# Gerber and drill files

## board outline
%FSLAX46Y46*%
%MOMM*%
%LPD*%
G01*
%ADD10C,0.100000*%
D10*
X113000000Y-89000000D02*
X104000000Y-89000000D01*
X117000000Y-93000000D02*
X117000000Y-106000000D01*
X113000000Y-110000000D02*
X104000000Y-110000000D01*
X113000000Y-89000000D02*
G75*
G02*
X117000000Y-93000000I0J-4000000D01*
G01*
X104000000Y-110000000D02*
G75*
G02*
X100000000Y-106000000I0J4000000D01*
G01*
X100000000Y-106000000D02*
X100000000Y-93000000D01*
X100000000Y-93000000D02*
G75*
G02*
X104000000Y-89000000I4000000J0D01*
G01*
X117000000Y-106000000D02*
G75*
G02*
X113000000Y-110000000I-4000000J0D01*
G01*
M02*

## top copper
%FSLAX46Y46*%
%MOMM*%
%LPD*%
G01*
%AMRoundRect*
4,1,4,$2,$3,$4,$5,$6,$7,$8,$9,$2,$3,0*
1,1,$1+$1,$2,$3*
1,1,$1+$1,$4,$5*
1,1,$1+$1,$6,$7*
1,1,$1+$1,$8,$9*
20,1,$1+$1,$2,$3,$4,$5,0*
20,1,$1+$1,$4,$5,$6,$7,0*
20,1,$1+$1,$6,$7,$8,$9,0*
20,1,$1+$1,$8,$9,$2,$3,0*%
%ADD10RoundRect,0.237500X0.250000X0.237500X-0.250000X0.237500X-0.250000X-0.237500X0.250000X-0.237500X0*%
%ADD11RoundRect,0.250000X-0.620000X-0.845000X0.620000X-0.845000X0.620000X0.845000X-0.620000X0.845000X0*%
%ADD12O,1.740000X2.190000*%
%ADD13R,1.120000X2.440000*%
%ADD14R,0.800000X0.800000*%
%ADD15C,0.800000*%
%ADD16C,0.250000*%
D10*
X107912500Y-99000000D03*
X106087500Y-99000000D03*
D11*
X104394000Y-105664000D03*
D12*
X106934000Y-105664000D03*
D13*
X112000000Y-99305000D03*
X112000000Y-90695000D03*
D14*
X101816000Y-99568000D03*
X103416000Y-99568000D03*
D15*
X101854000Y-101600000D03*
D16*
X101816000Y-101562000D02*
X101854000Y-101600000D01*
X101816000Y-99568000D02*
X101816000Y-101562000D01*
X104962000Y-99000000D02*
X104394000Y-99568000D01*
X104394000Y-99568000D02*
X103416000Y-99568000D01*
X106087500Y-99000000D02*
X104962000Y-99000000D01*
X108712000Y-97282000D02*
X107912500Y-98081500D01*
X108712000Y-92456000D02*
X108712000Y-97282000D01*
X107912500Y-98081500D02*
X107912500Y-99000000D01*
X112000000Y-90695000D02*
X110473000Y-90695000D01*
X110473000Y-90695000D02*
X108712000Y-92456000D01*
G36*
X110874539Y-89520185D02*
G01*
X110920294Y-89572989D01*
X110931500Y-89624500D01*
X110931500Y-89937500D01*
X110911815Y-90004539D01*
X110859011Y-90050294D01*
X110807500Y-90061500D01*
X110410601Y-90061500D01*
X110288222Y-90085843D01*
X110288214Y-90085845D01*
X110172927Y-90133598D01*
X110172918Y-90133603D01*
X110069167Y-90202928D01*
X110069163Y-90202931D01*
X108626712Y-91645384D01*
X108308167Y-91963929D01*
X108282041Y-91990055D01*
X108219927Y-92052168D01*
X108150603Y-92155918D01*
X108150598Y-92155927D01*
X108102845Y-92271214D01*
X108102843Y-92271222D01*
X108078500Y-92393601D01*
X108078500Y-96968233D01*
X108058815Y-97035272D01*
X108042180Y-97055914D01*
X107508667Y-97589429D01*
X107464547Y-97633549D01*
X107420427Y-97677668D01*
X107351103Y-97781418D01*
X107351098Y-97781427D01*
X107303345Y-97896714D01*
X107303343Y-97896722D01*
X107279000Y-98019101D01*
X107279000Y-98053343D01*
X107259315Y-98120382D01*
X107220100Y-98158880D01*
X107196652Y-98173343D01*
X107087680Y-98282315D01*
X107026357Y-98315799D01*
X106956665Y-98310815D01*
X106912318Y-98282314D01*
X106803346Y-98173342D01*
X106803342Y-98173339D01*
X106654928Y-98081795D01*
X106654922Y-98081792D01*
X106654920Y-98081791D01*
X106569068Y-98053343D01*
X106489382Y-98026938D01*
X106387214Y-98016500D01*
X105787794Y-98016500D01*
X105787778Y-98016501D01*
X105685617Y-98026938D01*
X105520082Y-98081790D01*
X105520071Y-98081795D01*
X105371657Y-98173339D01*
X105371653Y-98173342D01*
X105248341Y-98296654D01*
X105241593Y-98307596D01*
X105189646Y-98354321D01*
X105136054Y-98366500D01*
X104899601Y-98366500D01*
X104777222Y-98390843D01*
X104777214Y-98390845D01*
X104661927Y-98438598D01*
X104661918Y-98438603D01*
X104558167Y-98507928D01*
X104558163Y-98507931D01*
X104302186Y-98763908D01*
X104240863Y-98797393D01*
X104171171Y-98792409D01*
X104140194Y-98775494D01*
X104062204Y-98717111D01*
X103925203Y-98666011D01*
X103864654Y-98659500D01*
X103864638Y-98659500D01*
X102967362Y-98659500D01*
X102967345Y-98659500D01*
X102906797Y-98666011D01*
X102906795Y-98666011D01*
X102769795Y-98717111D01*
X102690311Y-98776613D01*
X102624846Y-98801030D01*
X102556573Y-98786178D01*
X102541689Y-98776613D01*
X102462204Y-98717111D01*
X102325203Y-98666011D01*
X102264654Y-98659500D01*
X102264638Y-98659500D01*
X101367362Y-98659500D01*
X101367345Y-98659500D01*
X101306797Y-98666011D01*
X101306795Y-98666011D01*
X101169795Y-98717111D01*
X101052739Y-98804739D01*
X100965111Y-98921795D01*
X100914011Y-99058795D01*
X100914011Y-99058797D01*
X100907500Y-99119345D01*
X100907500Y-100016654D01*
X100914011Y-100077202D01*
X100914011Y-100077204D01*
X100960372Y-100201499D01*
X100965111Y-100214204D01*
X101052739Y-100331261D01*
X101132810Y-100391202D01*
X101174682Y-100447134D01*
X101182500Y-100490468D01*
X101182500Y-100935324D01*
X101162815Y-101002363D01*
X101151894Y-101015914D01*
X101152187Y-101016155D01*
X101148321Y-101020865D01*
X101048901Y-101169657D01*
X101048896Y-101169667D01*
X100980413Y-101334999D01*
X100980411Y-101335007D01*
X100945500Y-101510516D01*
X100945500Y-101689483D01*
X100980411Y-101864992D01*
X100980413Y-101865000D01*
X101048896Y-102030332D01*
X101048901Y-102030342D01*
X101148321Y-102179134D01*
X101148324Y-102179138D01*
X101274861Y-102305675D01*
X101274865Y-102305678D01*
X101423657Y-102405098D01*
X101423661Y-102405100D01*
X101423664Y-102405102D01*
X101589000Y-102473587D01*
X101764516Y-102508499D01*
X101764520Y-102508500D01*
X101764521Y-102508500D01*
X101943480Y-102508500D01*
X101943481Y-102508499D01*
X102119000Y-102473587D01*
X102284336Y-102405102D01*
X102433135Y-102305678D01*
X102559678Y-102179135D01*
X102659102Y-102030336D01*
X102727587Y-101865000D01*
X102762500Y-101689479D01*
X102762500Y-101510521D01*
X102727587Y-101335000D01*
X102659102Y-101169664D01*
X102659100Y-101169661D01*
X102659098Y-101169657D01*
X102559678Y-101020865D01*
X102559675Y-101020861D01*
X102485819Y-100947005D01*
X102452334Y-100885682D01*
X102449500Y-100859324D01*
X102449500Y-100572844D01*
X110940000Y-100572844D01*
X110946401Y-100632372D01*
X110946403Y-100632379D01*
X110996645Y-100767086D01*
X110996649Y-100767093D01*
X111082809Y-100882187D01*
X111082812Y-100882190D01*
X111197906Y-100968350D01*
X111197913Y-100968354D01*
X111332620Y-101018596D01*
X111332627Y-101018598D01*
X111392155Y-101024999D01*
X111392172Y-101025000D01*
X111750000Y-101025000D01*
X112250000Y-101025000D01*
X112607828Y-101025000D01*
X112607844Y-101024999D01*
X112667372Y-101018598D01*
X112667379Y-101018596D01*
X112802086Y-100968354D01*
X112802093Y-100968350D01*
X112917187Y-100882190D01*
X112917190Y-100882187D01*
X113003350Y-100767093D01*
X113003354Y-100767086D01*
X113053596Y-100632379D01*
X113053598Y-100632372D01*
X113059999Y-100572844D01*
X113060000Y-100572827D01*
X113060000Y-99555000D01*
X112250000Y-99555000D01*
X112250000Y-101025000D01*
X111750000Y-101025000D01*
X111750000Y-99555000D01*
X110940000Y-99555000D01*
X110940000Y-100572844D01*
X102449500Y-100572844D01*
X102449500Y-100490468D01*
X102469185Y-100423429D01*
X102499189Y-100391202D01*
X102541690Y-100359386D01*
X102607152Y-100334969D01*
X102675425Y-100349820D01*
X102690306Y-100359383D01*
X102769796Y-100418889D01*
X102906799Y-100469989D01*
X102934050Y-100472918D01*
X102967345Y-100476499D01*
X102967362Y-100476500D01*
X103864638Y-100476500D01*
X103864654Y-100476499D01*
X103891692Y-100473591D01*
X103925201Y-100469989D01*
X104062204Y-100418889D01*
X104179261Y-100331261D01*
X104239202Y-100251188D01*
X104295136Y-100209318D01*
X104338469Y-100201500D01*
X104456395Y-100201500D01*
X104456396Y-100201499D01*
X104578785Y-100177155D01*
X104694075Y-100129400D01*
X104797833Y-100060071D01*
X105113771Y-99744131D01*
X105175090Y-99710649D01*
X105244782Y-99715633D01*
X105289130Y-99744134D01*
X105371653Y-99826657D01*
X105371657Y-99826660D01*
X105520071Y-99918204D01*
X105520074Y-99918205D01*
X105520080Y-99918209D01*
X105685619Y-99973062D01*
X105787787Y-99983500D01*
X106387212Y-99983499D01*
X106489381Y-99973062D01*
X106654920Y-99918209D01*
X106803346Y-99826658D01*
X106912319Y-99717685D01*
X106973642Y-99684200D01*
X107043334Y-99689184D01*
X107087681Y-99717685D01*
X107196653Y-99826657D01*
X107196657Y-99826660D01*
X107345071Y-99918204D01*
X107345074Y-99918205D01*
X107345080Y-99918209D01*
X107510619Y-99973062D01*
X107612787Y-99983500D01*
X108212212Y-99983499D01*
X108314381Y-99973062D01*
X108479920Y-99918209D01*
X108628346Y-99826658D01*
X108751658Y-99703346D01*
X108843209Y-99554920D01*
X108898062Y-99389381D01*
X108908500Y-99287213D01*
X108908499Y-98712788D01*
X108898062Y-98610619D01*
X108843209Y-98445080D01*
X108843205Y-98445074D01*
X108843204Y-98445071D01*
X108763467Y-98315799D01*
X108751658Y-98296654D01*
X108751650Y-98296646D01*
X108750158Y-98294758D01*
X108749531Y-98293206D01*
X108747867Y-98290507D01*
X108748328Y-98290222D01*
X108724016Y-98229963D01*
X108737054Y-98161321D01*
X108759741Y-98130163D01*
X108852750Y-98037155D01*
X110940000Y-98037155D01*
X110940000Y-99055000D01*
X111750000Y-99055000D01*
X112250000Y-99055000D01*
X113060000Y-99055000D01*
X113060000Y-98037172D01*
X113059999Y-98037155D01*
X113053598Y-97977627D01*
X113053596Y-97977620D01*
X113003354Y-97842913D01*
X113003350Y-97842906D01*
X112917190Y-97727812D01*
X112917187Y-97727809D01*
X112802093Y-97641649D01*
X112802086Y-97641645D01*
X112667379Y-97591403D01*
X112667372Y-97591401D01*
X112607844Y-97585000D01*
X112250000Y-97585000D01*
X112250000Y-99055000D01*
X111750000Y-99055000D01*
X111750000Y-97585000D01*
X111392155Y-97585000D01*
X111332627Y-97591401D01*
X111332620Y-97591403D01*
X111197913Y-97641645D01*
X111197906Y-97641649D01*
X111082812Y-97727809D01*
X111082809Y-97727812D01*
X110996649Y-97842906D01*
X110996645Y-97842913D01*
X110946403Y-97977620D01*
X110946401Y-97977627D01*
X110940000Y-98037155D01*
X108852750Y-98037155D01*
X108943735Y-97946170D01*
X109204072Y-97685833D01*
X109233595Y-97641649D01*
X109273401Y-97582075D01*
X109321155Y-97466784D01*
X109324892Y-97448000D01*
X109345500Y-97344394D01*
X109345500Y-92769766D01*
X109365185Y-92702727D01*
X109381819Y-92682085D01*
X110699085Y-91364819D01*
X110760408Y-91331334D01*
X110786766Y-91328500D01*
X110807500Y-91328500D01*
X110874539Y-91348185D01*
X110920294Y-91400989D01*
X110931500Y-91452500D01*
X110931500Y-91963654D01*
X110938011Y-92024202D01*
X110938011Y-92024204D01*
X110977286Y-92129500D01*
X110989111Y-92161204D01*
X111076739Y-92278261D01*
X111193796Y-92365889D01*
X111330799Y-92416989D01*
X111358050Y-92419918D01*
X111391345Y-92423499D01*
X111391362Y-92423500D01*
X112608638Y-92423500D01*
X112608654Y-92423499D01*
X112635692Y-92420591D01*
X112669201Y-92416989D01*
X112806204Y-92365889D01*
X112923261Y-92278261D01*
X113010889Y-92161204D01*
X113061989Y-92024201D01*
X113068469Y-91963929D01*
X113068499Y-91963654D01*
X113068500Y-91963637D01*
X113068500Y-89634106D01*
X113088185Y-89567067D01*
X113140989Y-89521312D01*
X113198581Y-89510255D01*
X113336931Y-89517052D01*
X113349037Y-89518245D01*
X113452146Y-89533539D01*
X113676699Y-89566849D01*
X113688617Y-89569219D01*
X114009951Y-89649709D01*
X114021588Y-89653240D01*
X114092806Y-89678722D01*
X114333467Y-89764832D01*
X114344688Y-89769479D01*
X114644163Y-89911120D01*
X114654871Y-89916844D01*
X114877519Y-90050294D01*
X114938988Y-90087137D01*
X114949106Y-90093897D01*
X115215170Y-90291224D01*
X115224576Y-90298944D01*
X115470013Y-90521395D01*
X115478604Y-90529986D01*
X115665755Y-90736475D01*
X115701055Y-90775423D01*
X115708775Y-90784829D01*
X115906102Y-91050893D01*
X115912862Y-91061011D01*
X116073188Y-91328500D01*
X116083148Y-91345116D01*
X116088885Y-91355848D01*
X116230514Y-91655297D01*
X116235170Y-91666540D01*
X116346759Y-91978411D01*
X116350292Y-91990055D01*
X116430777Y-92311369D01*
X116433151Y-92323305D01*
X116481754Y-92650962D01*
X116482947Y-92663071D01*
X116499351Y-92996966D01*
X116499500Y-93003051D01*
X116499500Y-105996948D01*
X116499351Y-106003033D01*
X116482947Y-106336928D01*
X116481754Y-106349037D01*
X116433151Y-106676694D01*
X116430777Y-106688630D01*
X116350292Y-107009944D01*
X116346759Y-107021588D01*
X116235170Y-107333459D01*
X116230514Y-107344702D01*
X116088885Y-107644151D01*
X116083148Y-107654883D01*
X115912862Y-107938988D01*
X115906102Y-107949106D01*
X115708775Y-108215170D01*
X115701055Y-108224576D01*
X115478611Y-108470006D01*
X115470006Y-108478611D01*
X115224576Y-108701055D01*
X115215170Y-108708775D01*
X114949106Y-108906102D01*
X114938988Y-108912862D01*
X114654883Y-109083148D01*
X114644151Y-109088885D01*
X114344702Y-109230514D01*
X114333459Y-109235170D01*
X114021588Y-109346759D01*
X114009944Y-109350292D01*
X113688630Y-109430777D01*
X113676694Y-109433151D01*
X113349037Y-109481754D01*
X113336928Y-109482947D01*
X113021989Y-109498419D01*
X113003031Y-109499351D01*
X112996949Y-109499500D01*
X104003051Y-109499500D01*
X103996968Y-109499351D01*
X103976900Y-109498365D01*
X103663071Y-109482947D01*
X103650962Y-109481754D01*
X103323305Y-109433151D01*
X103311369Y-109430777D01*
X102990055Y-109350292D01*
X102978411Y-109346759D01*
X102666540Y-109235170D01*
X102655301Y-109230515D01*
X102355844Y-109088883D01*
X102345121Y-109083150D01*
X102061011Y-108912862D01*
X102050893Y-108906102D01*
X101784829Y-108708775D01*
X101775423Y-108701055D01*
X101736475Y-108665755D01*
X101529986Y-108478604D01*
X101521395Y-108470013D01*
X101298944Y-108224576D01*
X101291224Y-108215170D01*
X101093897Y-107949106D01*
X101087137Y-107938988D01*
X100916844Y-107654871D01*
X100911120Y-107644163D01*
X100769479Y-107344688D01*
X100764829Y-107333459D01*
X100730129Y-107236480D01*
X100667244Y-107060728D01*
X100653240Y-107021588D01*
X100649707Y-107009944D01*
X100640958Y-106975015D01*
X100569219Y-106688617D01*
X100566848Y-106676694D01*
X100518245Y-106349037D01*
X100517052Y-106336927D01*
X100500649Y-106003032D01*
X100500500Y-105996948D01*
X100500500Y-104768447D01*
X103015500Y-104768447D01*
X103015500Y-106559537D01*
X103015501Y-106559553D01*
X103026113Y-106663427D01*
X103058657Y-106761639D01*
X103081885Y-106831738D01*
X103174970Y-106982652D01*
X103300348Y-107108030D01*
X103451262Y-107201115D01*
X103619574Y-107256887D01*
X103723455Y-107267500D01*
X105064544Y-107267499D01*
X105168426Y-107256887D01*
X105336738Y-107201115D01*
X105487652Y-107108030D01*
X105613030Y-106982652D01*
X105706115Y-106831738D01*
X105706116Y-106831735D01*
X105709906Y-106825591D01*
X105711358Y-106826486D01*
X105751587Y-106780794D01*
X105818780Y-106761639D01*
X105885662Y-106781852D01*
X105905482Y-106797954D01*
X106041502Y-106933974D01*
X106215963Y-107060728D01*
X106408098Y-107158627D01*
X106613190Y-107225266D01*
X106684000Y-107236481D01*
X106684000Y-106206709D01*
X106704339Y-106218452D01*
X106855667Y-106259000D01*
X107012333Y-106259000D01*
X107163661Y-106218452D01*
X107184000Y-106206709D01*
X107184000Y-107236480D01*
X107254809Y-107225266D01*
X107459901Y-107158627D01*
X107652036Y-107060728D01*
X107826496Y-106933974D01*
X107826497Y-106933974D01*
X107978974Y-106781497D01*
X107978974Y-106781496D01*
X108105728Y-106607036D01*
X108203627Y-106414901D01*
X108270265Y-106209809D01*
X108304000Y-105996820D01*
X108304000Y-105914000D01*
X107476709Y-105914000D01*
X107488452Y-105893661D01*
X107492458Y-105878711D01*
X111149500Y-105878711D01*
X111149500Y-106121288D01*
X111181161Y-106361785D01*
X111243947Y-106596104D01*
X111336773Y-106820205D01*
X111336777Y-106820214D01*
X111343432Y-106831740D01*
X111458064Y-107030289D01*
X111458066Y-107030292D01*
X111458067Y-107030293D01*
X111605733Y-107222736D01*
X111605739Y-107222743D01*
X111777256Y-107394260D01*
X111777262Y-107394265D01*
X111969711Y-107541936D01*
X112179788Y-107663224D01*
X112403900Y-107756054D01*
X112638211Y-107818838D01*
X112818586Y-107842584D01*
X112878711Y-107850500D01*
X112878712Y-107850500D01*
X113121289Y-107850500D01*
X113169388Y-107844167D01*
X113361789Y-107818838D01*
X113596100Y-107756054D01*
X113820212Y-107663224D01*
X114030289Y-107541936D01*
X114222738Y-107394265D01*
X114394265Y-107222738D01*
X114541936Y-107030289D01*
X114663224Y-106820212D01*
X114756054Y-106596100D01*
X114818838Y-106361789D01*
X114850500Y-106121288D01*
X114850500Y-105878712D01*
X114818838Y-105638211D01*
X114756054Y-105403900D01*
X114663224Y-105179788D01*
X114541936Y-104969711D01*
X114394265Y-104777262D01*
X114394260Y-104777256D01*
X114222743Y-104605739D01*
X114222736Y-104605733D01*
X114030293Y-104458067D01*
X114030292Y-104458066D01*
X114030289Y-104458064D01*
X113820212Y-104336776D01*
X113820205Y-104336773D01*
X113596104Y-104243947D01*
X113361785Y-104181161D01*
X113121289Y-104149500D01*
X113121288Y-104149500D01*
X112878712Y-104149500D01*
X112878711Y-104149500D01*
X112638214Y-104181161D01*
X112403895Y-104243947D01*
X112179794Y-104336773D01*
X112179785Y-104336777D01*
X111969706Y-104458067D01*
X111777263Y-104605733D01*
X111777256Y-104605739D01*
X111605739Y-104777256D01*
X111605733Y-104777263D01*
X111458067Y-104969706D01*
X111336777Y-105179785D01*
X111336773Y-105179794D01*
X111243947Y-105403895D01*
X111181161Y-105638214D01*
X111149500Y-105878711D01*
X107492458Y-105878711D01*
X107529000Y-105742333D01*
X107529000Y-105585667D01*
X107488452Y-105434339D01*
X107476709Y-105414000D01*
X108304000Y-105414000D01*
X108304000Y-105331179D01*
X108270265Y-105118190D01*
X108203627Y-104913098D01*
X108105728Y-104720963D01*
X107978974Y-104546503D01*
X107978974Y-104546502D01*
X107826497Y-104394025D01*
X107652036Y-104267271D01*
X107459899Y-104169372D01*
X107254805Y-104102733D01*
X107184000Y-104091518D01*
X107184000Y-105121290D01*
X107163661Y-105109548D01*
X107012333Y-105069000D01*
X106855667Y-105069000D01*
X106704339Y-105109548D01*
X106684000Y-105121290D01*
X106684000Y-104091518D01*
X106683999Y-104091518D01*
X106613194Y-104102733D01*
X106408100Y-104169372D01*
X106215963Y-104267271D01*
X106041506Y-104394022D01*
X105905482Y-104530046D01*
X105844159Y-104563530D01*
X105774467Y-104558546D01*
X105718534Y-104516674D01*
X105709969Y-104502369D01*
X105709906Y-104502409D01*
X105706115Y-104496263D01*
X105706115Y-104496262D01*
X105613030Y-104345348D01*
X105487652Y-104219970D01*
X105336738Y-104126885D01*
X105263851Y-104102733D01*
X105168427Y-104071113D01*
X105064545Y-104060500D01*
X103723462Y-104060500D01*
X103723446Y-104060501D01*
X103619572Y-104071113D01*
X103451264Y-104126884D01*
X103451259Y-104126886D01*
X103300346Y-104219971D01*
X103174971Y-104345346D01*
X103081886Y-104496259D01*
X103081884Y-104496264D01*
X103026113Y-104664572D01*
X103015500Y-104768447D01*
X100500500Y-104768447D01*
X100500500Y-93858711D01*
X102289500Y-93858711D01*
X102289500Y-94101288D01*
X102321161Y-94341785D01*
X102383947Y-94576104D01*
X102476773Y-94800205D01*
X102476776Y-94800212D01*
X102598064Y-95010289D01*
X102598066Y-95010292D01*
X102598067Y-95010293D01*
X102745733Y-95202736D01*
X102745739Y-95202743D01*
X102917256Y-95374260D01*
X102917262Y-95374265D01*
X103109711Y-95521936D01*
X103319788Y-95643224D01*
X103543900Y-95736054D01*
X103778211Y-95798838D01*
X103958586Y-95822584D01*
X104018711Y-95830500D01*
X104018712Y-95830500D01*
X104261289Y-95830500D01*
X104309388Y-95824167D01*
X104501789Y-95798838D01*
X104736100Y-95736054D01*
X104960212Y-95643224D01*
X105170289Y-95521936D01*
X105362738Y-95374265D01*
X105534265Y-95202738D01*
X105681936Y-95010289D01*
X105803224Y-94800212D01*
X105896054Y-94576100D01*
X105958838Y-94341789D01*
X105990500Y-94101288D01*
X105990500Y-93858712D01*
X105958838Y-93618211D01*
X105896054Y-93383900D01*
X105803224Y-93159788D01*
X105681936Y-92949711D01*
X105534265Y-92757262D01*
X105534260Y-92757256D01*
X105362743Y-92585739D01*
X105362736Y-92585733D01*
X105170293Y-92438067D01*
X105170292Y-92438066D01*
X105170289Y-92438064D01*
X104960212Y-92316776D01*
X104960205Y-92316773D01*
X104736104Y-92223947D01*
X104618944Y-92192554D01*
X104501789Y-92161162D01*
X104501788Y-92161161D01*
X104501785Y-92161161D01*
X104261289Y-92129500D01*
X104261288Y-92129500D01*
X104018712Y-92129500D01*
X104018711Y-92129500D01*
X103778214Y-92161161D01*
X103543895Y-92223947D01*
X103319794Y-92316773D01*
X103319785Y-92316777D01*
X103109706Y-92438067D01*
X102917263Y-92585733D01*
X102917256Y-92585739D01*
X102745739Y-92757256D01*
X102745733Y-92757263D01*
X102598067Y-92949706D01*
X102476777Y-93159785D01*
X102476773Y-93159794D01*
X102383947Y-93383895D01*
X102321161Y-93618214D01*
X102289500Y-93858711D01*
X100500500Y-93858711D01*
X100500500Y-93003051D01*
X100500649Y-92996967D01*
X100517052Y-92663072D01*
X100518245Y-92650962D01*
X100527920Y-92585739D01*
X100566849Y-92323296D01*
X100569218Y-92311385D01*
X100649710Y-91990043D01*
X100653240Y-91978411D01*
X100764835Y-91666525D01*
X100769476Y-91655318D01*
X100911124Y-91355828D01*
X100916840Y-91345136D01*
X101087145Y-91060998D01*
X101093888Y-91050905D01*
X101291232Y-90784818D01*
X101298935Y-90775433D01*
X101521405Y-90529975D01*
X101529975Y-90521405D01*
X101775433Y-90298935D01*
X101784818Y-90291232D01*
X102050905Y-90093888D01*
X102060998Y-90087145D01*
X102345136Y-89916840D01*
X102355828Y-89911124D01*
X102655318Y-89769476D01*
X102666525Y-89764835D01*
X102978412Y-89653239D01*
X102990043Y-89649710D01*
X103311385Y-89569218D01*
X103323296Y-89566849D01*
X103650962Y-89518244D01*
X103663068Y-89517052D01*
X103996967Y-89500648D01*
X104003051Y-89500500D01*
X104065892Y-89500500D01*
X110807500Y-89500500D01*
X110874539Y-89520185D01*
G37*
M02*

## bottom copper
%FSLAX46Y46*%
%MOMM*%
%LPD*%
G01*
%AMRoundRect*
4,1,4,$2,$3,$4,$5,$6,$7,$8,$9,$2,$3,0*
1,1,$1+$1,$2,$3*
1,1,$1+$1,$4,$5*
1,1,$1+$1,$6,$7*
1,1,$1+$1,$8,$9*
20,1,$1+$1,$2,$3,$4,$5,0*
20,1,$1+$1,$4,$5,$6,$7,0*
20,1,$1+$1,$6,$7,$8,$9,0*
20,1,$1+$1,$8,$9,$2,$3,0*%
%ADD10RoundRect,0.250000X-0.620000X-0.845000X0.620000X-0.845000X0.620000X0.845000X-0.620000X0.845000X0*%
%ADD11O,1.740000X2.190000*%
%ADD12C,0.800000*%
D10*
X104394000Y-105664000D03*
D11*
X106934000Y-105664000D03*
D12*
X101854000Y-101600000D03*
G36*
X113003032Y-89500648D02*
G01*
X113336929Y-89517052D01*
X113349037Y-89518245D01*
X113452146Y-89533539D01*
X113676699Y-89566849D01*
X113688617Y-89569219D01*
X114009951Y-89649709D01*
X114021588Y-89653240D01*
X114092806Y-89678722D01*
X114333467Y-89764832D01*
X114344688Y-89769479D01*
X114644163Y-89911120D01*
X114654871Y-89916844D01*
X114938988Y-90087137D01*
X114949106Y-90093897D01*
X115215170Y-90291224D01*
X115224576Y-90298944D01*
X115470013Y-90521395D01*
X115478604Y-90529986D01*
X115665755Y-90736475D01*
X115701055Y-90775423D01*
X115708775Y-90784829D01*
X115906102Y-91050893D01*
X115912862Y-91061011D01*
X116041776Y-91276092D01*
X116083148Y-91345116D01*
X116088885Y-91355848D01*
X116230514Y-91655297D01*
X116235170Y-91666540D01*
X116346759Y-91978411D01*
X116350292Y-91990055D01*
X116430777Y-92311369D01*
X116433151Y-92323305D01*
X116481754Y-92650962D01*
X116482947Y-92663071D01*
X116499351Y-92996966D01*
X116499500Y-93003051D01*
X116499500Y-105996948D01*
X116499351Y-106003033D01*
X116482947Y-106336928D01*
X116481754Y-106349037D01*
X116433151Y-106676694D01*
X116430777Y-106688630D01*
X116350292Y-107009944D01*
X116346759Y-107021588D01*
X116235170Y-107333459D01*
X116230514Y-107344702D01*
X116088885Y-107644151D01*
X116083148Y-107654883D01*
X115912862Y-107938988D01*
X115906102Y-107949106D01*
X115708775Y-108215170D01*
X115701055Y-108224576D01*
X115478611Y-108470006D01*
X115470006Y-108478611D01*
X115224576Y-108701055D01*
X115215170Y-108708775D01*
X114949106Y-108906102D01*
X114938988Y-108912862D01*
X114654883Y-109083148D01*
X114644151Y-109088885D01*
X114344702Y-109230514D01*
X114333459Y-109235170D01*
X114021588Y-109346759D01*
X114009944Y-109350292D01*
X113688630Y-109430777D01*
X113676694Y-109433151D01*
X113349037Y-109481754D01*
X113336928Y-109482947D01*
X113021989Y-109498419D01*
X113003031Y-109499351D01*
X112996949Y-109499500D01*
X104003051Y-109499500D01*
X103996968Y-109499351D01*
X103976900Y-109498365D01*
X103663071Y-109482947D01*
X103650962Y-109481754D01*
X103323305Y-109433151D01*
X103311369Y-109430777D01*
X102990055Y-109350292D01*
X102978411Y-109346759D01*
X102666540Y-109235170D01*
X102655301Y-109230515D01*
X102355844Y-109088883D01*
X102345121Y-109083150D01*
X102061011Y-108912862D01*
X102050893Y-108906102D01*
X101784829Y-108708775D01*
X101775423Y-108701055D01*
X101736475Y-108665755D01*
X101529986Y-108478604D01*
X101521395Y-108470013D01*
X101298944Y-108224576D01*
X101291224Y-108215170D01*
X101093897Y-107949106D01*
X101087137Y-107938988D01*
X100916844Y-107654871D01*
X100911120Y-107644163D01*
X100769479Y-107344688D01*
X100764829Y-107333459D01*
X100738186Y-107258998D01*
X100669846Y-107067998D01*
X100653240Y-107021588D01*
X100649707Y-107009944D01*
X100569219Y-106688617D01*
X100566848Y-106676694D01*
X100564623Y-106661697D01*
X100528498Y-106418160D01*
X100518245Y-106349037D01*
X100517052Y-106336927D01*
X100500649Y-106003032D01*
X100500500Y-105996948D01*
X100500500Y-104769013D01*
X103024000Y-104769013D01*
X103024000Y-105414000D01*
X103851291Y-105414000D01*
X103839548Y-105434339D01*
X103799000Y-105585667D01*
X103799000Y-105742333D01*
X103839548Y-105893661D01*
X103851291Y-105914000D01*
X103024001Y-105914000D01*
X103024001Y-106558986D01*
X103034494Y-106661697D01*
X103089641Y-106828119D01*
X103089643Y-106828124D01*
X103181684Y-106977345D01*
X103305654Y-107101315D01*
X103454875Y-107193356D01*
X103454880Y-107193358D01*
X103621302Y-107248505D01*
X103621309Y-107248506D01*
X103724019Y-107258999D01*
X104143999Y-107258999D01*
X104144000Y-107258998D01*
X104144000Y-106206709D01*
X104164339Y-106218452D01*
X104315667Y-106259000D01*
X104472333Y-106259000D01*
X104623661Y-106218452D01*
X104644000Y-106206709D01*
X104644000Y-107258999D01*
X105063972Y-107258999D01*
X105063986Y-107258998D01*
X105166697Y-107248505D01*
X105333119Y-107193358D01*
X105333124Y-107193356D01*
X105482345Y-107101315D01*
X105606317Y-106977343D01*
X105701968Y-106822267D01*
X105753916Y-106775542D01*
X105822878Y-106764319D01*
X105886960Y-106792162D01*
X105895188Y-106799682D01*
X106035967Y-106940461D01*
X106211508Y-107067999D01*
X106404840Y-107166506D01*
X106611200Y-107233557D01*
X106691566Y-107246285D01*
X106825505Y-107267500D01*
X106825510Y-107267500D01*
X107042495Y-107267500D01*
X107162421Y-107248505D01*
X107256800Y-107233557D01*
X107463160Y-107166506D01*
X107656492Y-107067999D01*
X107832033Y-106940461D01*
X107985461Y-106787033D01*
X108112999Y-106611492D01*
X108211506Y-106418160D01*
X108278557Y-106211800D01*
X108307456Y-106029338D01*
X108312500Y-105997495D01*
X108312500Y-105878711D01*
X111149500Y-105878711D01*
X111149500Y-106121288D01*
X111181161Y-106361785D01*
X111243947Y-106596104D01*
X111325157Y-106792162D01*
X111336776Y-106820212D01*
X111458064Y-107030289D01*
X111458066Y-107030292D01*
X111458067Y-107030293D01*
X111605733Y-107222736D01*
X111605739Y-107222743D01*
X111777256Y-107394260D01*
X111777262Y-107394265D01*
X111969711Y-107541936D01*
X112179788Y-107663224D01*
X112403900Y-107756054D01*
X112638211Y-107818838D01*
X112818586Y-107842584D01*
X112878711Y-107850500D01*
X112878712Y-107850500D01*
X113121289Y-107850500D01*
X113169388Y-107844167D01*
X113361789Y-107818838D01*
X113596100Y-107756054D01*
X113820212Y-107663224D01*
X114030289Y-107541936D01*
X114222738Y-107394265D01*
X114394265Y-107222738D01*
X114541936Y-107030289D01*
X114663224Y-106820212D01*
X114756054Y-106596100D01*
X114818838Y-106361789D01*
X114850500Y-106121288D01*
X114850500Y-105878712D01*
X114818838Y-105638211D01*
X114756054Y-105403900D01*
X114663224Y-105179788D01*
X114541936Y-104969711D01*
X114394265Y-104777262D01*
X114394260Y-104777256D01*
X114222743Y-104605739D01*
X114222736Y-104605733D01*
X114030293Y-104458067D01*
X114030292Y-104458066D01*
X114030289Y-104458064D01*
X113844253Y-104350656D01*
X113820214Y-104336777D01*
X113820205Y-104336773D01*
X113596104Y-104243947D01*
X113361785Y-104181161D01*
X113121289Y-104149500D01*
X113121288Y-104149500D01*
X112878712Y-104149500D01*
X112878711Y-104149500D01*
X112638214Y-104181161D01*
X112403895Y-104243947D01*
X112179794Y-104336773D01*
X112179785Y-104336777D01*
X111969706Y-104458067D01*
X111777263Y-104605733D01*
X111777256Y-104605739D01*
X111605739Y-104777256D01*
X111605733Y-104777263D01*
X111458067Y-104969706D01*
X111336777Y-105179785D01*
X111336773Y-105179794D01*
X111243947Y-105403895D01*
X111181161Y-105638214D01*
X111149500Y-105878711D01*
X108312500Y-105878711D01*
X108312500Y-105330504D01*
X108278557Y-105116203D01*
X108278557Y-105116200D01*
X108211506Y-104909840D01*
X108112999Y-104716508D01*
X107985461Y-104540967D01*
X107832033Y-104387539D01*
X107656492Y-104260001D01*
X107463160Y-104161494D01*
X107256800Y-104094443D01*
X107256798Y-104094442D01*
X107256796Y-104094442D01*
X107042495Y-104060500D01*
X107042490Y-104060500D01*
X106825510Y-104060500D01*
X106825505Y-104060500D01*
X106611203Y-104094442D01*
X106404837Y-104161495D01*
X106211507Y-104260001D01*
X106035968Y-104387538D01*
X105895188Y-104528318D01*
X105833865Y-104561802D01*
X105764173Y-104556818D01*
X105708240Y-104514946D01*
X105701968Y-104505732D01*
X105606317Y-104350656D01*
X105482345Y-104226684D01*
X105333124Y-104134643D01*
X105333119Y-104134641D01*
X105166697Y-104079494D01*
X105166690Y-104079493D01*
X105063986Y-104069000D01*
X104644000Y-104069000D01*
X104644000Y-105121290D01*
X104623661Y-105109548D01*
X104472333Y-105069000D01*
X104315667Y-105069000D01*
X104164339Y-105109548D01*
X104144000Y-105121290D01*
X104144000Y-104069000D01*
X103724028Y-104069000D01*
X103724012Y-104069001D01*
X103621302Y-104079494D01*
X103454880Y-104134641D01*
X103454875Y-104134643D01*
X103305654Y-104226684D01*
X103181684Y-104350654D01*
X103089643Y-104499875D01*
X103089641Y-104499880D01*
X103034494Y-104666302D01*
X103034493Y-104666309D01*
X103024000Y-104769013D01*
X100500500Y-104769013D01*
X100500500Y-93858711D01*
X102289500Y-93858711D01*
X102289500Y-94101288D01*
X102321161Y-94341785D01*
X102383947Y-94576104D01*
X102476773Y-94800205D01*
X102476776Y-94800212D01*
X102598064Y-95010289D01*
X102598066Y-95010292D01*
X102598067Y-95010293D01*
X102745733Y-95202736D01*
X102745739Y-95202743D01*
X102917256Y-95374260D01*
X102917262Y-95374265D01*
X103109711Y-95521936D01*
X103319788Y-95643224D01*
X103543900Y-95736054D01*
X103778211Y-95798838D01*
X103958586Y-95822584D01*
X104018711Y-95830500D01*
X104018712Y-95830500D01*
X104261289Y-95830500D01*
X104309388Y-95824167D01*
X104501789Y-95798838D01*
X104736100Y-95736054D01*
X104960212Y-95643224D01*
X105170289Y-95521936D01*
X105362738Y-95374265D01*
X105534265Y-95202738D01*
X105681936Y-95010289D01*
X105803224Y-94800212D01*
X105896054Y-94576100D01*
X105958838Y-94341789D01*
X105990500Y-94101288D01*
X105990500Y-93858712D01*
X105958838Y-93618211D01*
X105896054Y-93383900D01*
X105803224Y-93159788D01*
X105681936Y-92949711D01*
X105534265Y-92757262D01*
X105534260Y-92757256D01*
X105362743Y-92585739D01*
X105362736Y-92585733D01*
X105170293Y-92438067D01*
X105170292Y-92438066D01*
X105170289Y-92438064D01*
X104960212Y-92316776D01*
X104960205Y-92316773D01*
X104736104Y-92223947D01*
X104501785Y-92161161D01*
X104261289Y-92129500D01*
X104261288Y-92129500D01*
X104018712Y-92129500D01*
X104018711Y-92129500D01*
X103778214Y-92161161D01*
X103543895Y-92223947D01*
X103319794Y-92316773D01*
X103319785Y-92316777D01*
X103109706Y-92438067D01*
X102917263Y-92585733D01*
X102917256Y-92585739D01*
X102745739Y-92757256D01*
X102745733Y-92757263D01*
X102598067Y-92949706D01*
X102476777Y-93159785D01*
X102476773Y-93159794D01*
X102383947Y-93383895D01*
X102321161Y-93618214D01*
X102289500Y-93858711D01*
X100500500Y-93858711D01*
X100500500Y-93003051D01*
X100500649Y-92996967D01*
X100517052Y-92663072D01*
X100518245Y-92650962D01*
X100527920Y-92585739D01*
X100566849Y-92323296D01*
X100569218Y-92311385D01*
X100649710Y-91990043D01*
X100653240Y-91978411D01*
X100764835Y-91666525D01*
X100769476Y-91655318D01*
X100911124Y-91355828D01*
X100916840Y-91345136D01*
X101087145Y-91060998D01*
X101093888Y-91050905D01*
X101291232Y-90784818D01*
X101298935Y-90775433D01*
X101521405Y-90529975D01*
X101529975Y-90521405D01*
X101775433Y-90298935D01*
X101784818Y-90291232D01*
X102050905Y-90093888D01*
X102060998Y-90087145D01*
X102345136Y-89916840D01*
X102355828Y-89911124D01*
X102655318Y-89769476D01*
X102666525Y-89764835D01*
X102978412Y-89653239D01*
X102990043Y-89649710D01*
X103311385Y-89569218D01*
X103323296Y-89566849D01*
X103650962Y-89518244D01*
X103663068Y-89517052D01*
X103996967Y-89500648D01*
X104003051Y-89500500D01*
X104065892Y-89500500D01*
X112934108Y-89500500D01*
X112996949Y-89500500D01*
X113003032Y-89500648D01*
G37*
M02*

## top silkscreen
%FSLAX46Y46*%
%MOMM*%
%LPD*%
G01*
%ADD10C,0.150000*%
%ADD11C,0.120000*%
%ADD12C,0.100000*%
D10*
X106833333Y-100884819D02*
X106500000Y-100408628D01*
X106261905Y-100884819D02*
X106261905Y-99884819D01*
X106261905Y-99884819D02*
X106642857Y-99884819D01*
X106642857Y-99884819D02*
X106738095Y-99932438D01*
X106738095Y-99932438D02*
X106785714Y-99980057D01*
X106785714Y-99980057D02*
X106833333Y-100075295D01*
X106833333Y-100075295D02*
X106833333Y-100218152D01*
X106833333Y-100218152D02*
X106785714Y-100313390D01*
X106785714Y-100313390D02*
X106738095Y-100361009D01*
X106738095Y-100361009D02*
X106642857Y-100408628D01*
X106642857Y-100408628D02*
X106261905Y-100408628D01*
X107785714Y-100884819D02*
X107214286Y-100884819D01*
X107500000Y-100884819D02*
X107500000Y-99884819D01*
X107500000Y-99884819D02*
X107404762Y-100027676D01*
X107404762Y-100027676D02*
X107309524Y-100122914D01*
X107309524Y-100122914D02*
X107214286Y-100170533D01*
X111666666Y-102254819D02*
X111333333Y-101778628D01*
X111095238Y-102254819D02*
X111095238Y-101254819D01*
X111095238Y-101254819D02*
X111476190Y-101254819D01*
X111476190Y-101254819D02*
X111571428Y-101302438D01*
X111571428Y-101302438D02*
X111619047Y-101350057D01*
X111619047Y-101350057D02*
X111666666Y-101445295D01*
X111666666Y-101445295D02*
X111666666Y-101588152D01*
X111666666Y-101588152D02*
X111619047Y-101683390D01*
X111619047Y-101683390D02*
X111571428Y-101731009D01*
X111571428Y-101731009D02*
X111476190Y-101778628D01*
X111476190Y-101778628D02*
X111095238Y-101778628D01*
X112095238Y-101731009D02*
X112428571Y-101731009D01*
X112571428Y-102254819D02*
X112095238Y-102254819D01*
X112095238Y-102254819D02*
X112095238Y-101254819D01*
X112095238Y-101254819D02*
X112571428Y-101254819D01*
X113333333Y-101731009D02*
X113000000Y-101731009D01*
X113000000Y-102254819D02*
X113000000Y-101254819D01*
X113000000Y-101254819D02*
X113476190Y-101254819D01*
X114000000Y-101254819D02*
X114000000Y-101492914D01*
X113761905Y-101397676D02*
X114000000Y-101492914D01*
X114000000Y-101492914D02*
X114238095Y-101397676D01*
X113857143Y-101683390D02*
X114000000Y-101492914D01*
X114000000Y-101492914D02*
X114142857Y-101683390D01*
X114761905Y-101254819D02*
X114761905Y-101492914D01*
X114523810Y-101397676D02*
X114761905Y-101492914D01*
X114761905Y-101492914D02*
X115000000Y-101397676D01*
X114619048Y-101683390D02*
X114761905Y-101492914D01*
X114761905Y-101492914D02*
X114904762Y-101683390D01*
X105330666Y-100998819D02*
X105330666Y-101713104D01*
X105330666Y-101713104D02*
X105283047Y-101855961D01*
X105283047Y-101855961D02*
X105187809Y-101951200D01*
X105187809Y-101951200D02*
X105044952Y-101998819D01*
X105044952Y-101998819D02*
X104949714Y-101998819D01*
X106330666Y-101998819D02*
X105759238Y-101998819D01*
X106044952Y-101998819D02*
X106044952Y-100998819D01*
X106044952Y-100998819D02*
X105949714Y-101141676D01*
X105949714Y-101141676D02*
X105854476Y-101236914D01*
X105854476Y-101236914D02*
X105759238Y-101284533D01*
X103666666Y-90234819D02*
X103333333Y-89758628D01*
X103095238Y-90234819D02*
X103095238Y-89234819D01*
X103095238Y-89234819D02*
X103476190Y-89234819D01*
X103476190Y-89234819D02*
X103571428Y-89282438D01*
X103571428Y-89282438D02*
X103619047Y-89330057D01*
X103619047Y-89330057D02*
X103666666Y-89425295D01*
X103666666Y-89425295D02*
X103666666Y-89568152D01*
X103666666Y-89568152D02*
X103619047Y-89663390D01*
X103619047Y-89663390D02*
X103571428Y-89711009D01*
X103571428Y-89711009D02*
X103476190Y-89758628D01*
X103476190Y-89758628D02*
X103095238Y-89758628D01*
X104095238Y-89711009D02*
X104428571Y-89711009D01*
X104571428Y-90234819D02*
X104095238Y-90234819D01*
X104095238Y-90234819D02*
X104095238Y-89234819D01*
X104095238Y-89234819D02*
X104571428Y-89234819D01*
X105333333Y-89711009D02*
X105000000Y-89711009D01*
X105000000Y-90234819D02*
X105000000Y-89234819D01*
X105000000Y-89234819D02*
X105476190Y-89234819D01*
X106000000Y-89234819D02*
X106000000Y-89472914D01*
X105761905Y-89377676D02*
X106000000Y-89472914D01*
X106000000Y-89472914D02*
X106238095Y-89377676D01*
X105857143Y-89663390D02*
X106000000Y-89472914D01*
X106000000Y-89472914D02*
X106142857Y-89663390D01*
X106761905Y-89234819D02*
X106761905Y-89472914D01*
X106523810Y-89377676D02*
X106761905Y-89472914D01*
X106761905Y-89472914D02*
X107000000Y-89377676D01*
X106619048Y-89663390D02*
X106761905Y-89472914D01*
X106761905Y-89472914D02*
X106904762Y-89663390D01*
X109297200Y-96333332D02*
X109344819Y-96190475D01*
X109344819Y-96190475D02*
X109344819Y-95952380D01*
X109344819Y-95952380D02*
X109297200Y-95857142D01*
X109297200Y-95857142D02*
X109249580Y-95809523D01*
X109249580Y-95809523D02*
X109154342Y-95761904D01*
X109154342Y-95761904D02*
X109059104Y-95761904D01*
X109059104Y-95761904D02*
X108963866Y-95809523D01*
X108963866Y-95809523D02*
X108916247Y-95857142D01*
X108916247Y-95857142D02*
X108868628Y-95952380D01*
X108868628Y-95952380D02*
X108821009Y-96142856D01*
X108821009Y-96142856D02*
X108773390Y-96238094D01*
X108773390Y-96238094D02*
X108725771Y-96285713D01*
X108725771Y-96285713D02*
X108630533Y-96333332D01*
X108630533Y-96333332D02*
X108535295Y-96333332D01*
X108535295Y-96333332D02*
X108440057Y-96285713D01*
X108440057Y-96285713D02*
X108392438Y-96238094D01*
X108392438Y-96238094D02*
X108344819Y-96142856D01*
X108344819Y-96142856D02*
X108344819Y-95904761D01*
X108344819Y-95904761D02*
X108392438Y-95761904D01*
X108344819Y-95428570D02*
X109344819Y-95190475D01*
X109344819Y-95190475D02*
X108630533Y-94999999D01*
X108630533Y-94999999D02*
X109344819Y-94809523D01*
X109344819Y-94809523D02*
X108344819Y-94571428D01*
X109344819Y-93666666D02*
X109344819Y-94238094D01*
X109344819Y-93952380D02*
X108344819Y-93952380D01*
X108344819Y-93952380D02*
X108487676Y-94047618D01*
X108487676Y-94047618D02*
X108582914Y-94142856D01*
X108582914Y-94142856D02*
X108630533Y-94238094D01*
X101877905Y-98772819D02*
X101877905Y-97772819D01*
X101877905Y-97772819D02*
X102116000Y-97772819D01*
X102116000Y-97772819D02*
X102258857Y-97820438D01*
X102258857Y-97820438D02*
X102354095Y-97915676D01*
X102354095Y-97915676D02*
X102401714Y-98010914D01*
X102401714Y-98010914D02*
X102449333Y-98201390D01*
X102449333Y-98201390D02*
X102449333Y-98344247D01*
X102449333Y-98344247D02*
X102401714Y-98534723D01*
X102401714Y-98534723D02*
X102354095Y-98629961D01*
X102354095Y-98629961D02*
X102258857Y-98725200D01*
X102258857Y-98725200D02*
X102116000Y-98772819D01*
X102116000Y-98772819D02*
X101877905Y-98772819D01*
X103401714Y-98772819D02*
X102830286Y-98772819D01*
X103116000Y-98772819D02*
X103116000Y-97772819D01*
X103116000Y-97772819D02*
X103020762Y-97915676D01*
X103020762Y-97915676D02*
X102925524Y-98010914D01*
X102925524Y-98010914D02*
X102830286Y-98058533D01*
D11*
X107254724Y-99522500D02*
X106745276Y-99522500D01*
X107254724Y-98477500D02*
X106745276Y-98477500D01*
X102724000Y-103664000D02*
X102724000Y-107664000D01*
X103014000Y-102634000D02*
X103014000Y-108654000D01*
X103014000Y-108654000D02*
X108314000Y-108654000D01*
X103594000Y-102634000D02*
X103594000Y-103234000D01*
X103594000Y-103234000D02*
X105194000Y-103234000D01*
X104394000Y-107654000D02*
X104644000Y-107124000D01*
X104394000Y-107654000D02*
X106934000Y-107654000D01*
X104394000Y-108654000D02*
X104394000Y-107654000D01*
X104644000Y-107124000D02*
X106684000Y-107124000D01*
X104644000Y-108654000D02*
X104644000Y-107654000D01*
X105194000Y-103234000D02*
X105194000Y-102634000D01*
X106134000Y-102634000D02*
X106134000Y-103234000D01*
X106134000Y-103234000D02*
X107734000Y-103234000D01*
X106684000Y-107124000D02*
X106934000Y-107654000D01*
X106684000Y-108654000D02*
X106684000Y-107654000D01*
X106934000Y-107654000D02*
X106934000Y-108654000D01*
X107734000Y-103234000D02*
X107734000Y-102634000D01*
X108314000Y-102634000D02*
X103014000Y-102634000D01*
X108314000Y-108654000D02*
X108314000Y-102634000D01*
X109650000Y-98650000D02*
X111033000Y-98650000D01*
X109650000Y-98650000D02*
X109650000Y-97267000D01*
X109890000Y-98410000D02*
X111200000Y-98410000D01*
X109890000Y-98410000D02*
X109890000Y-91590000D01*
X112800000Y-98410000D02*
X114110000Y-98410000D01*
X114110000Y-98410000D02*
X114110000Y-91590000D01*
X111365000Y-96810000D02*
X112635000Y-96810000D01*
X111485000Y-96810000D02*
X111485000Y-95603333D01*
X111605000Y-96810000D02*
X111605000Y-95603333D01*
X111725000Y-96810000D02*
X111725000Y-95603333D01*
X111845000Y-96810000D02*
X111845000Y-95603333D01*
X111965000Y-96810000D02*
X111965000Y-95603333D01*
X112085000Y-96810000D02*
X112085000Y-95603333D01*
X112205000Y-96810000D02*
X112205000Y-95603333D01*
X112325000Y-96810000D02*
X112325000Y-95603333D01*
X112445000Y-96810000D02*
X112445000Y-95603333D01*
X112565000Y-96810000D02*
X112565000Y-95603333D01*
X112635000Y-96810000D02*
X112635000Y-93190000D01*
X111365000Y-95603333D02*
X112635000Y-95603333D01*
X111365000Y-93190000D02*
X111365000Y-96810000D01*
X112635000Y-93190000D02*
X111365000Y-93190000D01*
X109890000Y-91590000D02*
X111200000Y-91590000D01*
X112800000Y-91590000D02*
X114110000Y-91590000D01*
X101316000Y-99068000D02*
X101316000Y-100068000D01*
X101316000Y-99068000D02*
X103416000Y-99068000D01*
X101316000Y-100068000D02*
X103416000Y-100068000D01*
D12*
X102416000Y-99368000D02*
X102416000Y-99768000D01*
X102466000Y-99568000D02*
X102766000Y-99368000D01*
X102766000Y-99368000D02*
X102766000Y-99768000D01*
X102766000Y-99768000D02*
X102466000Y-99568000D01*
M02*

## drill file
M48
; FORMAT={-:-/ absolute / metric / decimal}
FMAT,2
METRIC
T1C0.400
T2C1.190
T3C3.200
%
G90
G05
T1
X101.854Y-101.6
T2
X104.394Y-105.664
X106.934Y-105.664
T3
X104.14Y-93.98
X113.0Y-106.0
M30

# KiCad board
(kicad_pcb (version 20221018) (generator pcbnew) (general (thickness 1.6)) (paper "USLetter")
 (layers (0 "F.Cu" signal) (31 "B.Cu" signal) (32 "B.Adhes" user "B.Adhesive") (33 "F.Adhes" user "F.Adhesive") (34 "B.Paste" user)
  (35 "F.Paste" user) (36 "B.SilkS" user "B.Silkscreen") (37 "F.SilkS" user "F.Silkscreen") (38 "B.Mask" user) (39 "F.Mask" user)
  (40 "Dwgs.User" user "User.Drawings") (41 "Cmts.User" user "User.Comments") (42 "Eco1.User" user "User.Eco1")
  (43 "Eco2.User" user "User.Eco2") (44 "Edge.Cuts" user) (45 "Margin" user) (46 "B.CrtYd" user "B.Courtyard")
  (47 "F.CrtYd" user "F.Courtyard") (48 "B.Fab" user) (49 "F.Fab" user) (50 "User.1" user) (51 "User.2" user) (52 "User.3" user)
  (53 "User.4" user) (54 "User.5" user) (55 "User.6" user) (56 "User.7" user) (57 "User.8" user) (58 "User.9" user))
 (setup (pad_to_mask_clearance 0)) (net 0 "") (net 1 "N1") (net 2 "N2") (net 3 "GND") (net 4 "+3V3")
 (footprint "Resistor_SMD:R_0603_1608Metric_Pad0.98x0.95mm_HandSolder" (layer "F.Cu") (at 107 99 180)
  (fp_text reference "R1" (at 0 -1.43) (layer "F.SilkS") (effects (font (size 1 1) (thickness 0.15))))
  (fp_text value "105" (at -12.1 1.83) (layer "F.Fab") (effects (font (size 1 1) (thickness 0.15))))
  (fp_line (start -0.254724 -0.5225) (end 0.254724 -0.5225) (stroke (width 0.12) (type solid)) (layer "F.SilkS"))
  (fp_line (start -0.254724 0.5225) (end 0.254724 0.5225) (stroke (width 0.12) (type solid)) (layer "F.SilkS"))
  (pad "1" smd roundrect (at -0.9125 0 180) (size 0.975 0.95) (layers "F.Cu" "F.Paste" "F.Mask") (roundrect_rratio 0.25) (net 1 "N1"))
  (pad "2" smd roundrect (at 0.9125 0 180) (size 0.975 0.95) (layers "F.Cu" "F.Paste" "F.Mask") (roundrect_rratio 0.25) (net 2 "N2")))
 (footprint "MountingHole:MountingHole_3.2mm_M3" (layer "F.Cu") (at 113 106)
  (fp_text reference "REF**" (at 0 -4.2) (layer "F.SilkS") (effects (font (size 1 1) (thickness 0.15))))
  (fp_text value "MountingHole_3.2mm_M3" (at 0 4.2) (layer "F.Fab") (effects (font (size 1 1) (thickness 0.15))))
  (pad "" np_thru_hole circle (at 0 0) (size 3.2 3.2) (drill 3.2) (layers "F&B.Cu" "*.Mask")))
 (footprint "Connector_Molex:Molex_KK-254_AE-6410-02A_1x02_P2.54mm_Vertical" (layer "F.Cu") (at 104.394 105.664)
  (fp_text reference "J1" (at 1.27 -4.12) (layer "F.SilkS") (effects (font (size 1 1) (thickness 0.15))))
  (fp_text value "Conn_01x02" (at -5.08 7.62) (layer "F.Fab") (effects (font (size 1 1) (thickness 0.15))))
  (fp_line (start -1.67 -2) (end -1.67 2) (stroke (width 0.12) (type solid)) (layer "F.SilkS"))
  (fp_line (start -1.38 -3.03) (end -1.38 2.99) (stroke (width 0.12) (type solid)) (layer "F.SilkS"))
  (fp_line (start -1.38 2.99) (end 3.92 2.99) (stroke (width 0.12) (type solid)) (layer "F.SilkS"))
  (fp_line (start -0.8 -3.03) (end -0.8 -2.43) (stroke (width 0.12) (type solid)) (layer "F.SilkS"))
  (fp_line (start -0.8 -2.43) (end 0.8 -2.43) (stroke (width 0.12) (type solid)) (layer "F.SilkS"))
  (fp_line (start 0 1.99) (end 0.25 1.46) (stroke (width 0.12) (type solid)) (layer "F.SilkS"))
  (fp_line (start 0 1.99) (end 2.54 1.99) (stroke (width 0.12) (type solid)) (layer "F.SilkS"))
  (fp_line (start 0 2.99) (end 0 1.99) (stroke (width 0.12) (type solid)) (layer "F.SilkS"))
  (fp_line (start 0.25 1.46) (end 2.29 1.46) (stroke (width 0.12) (type solid)) (layer "F.SilkS"))
  (fp_line (start 0.25 2.99) (end 0.25 1.99) (stroke (width 0.12) (type solid)) (layer "F.SilkS"))
  (fp_line (start 0.8 -2.43) (end 0.8 -3.03) (stroke (width 0.12) (type solid)) (layer "F.SilkS"))
  (fp_line (start 1.74 -3.03) (end 1.74 -2.43) (stroke (width 0.12) (type solid)) (layer "F.SilkS"))
  (fp_line (start 1.74 -2.43) (end 3.34 -2.43) (stroke (width 0.12) (type solid)) (layer "F.SilkS"))
  (fp_line (start 2.29 1.46) (end 2.54 1.99) (stroke (width 0.12) (type solid)) (layer "F.SilkS"))
  (fp_line (start 2.29 2.99) (end 2.29 1.99) (stroke (width 0.12) (type solid)) (layer "F.SilkS"))
  (fp_line (start 2.54 1.99) (end 2.54 2.99) (stroke (width 0.12) (type solid)) (layer "F.SilkS"))
  (fp_line (start 3.34 -2.43) (end 3.34 -3.03) (stroke (width 0.12) (type solid)) (layer "F.SilkS"))
  (fp_line (start 3.92 -3.03) (end -1.38 -3.03) (stroke (width 0.12) (type solid)) (layer "F.SilkS"))
  (fp_line (start 3.92 2.99) (end 3.92 -3.03) (stroke (width 0.12) (type solid)) (layer "F.SilkS"))
  (pad "1" thru_hole roundrect (at 0 0) (size 1.74 2.19) (drill 1.19) (layers "*.Cu" "*.Mask") (roundrect_rratio 0.143678) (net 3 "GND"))
  (pad "2" thru_hole oval (at 2.54 0) (size 1.74 2.19) (drill 1.19) (layers "*.Cu" "*.Mask") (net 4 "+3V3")))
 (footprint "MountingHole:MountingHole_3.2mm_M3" (layer "F.Cu") (at 104.14 93.98)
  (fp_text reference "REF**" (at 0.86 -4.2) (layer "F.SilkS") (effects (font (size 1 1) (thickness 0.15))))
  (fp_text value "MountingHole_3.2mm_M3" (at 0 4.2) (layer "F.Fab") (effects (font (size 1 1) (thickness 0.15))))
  (pad "" np_thru_hole circle (at 0 0) (size 3.2 3.2) (drill 3.2) (layers "*.Cu" "*.Mask")))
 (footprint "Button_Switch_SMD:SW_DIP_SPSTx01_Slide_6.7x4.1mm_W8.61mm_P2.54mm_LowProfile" (layer "F.Cu") (at 112 95 90)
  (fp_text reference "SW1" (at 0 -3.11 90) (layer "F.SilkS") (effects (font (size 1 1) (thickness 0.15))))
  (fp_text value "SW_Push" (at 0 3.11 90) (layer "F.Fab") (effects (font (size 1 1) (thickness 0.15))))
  (fp_line (start -3.65 -2.35) (end -3.65 -0.967) (stroke (width 0.12) (type solid)) (layer "F.SilkS"))
  (fp_line (start -3.65 -2.35) (end -2.267 -2.35) (stroke (width 0.12) (type solid)) (layer "F.SilkS"))
  (fp_line (start -3.41 -2.11) (end -3.41 -0.8) (stroke (width 0.12) (type solid)) (layer "F.SilkS"))
  (fp_line (start -3.41 -2.11) (end 3.41 -2.11) (stroke (width 0.12) (type solid)) (layer "F.SilkS"))
  (fp_line (start -3.41 0.8) (end -3.41 2.11) (stroke (width 0.12) (type solid)) (layer "F.SilkS"))
  (fp_line (start -3.41 2.11) (end 3.41 2.11) (stroke (width 0.12) (type solid)) (layer "F.SilkS"))
  (fp_line (start -1.81 -0.635) (end -1.81 0.635) (stroke (width 0.12) (type solid)) (layer "F.SilkS"))
  (fp_line (start -1.81 -0.515) (end -0.603333 -0.515) (stroke (width 0.12) (type solid)) (layer "F.SilkS"))
  (fp_line (start -1.81 -0.395) (end -0.603333 -0.395) (stroke (width 0.12) (type solid)) (layer "F.SilkS"))
  (fp_line (start -1.81 -0.275) (end -0.603333 -0.275) (stroke (width 0.12) (type solid)) (layer "F.SilkS"))
  (fp_line (start -1.81 -0.155) (end -0.603333 -0.155) (stroke (width 0.12) (type solid)) (layer "F.SilkS"))
  (fp_line (start -1.81 -0.035) (end -0.603333 -0.035) (stroke (width 0.12) (type solid)) (layer "F.SilkS"))
  (fp_line (start -1.81 0.085) (end -0.603333 0.085) (stroke (width 0.12) (type solid)) (layer "F.SilkS"))
  (fp_line (start -1.81 0.205) (end -0.603333 0.205) (stroke (width 0.12) (type solid)) (layer "F.SilkS"))
  (fp_line (start -1.81 0.325) (end -0.603333 0.325) (stroke (width 0.12) (type solid)) (layer "F.SilkS"))
  (fp_line (start -1.81 0.445) (end -0.603333 0.445) (stroke (width 0.12) (type solid)) (layer "F.SilkS"))
  (fp_line (start -1.81 0.565) (end -0.603333 0.565) (stroke (width 0.12) (type solid)) (layer "F.SilkS"))
  (fp_line (start -1.81 0.635) (end 1.81 0.635) (stroke (width 0.12) (type solid)) (layer "F.SilkS"))
  (fp_line (start -0.603333 -0.635) (end -0.603333 0.635) (stroke (width 0.12) (type solid)) (layer "F.SilkS"))
  (fp_line (start 1.81 -0.635) (end -1.81 -0.635) (stroke (width 0.12) (type solid)) (layer "F.SilkS"))
  (fp_line (start 1.81 0.635) (end 1.81 -0.635) (stroke (width 0.12) (type solid)) (layer "F.SilkS"))
  (fp_line (start 3.41 -2.11) (end 3.41 -0.8) (stroke (width 0.12) (type solid)) (layer "F.SilkS"))
  (fp_line (start 3.41 0.8) (end 3.41 2.11) (stroke (width 0.12) (type solid)) (layer "F.SilkS"))
  (pad "1" smd rect (at -4.305 0 90) (size 2.44 1.12) (layers "F.Cu" "F.Paste" "F.Mask") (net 4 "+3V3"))
  (pad "2" smd rect (at 4.305 0 90) (size 2.44 1.12) (layers "F.Cu" "F.Paste" "F.Mask") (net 1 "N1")))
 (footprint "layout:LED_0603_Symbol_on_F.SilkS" (layer "F.Cu") (at 102.616 99.568)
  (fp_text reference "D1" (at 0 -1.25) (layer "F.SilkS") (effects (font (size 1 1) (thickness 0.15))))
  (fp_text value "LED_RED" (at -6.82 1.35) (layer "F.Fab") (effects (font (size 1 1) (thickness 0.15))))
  (fp_line (start -1.3 -0.5) (end -1.3 0.5) (stroke (width 0.12) (type solid)) (layer "F.SilkS"))
  (fp_line (start -1.3 -0.5) (end 0.8 -0.5) (stroke (width 0.12) (type solid)) (layer "F.SilkS"))
  (fp_line (start -1.3 0.5) (end 0.8 0.5) (stroke (width 0.12) (type solid)) (layer "F.SilkS"))
  (fp_line (start -0.2 -0.2) (end -0.2 0.2) (stroke (width 0.1) (type solid)) (layer "F.SilkS"))
  (fp_line (start -0.15 0) (end 0.15 -0.2) (stroke (width 0.1) (type solid)) (layer "F.SilkS"))
  (fp_line (start 0.15 -0.2) (end 0.15 0.2) (stroke (width 0.1) (type solid)) (layer "F.SilkS"))
  (fp_line (start 0.15 0.2) (end -0.15 0) (stroke (width 0.1) (type solid)) (layer "F.SilkS"))
  (pad "1" smd rect (at -0.8 0 180) (size 0.8 0.8) (layers "F.Cu" "F.Paste" "F.Mask") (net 3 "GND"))
  (pad "2" smd rect (at 0.8 0 180) (size 0.8 0.8) (layers "F.Cu" "F.Paste" "F.Mask") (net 2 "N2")))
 (gr_line (start 113 89) (end 104 89) (stroke (width 0.1) (type default)) (layer "Edge.Cuts"))
 (gr_line (start 117 93) (end 117 106) (stroke (width 0.1) (type default)) (layer "Edge.Cuts"))
 (gr_line (start 113 110) (end 104 110) (stroke (width 0.1) (type default)) (layer "Edge.Cuts"))
 (gr_arc (start 113 89) (mid 115.828427 90.171573) (end 117 93) (stroke (width 0.1) (type default)) (layer "Edge.Cuts"))
 (gr_arc (start 104 110) (mid 101.171573 108.828427) (end 100 106) (stroke (width 0.1) (type default)) (layer "Edge.Cuts"))
 (gr_line (start 100 106) (end 100 93) (stroke (width 0.1) (type default)) (layer "Edge.Cuts"))
 (gr_arc (start 100 93) (mid 101.171573 90.171573) (end 104 89) (stroke (width 0.1) (type default)) (layer "Edge.Cuts"))
 (gr_arc (start 117 106) (mid 115.828427 108.828427) (end 113 110) (stroke (width 0.1) (type default)) (layer "Edge.Cuts"))
 (segment (start 101.816 101.562) (end 101.854 101.6) (width 0.25) (layer "F.Cu") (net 3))
 (segment (start 101.816 99.568) (end 101.816 101.562) (width 0.25) (layer "F.Cu") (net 3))
 (via (at 101.854 101.6) (size 0.8) (drill 0.4) (layers "F.Cu" "B.Cu") (free) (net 3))
 (segment (start 104.962 99) (end 104.394 99.568) (width 0.25) (layer "F.Cu") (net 2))
 (segment (start 104.394 99.568) (end 103.416 99.568) (width 0.25) (layer "F.Cu") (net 2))
 (segment (start 106.0875 99) (end 104.962 99) (width 0.25) (layer "F.Cu") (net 2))
 (segment (start 108.712 97.282) (end 107.9125 98.0815) (width 0.25) (layer "F.Cu") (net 1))
 (segment (start 108.712 92.456) (end 108.712 97.282) (width 0.25) (layer "F.Cu") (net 1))
 (segment (start 107.9125 98.0815) (end 107.9125 99) (width 0.25) (layer "F.Cu") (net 1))
 (segment (start 112 90.695) (end 110.473 90.695) (width 0.25) (layer "F.Cu") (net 1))
 (segment (start 110.473 90.695) (end 108.712 92.456) (width 0.25) (layer "F.Cu") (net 1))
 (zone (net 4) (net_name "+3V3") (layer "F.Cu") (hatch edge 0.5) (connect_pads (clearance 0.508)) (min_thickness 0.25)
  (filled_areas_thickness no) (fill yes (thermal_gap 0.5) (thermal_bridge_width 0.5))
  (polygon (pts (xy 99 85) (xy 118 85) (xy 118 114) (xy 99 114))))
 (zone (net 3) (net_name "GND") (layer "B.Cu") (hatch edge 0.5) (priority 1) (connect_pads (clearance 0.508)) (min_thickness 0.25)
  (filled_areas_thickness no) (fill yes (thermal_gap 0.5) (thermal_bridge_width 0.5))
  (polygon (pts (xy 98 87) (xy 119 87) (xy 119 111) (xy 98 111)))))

